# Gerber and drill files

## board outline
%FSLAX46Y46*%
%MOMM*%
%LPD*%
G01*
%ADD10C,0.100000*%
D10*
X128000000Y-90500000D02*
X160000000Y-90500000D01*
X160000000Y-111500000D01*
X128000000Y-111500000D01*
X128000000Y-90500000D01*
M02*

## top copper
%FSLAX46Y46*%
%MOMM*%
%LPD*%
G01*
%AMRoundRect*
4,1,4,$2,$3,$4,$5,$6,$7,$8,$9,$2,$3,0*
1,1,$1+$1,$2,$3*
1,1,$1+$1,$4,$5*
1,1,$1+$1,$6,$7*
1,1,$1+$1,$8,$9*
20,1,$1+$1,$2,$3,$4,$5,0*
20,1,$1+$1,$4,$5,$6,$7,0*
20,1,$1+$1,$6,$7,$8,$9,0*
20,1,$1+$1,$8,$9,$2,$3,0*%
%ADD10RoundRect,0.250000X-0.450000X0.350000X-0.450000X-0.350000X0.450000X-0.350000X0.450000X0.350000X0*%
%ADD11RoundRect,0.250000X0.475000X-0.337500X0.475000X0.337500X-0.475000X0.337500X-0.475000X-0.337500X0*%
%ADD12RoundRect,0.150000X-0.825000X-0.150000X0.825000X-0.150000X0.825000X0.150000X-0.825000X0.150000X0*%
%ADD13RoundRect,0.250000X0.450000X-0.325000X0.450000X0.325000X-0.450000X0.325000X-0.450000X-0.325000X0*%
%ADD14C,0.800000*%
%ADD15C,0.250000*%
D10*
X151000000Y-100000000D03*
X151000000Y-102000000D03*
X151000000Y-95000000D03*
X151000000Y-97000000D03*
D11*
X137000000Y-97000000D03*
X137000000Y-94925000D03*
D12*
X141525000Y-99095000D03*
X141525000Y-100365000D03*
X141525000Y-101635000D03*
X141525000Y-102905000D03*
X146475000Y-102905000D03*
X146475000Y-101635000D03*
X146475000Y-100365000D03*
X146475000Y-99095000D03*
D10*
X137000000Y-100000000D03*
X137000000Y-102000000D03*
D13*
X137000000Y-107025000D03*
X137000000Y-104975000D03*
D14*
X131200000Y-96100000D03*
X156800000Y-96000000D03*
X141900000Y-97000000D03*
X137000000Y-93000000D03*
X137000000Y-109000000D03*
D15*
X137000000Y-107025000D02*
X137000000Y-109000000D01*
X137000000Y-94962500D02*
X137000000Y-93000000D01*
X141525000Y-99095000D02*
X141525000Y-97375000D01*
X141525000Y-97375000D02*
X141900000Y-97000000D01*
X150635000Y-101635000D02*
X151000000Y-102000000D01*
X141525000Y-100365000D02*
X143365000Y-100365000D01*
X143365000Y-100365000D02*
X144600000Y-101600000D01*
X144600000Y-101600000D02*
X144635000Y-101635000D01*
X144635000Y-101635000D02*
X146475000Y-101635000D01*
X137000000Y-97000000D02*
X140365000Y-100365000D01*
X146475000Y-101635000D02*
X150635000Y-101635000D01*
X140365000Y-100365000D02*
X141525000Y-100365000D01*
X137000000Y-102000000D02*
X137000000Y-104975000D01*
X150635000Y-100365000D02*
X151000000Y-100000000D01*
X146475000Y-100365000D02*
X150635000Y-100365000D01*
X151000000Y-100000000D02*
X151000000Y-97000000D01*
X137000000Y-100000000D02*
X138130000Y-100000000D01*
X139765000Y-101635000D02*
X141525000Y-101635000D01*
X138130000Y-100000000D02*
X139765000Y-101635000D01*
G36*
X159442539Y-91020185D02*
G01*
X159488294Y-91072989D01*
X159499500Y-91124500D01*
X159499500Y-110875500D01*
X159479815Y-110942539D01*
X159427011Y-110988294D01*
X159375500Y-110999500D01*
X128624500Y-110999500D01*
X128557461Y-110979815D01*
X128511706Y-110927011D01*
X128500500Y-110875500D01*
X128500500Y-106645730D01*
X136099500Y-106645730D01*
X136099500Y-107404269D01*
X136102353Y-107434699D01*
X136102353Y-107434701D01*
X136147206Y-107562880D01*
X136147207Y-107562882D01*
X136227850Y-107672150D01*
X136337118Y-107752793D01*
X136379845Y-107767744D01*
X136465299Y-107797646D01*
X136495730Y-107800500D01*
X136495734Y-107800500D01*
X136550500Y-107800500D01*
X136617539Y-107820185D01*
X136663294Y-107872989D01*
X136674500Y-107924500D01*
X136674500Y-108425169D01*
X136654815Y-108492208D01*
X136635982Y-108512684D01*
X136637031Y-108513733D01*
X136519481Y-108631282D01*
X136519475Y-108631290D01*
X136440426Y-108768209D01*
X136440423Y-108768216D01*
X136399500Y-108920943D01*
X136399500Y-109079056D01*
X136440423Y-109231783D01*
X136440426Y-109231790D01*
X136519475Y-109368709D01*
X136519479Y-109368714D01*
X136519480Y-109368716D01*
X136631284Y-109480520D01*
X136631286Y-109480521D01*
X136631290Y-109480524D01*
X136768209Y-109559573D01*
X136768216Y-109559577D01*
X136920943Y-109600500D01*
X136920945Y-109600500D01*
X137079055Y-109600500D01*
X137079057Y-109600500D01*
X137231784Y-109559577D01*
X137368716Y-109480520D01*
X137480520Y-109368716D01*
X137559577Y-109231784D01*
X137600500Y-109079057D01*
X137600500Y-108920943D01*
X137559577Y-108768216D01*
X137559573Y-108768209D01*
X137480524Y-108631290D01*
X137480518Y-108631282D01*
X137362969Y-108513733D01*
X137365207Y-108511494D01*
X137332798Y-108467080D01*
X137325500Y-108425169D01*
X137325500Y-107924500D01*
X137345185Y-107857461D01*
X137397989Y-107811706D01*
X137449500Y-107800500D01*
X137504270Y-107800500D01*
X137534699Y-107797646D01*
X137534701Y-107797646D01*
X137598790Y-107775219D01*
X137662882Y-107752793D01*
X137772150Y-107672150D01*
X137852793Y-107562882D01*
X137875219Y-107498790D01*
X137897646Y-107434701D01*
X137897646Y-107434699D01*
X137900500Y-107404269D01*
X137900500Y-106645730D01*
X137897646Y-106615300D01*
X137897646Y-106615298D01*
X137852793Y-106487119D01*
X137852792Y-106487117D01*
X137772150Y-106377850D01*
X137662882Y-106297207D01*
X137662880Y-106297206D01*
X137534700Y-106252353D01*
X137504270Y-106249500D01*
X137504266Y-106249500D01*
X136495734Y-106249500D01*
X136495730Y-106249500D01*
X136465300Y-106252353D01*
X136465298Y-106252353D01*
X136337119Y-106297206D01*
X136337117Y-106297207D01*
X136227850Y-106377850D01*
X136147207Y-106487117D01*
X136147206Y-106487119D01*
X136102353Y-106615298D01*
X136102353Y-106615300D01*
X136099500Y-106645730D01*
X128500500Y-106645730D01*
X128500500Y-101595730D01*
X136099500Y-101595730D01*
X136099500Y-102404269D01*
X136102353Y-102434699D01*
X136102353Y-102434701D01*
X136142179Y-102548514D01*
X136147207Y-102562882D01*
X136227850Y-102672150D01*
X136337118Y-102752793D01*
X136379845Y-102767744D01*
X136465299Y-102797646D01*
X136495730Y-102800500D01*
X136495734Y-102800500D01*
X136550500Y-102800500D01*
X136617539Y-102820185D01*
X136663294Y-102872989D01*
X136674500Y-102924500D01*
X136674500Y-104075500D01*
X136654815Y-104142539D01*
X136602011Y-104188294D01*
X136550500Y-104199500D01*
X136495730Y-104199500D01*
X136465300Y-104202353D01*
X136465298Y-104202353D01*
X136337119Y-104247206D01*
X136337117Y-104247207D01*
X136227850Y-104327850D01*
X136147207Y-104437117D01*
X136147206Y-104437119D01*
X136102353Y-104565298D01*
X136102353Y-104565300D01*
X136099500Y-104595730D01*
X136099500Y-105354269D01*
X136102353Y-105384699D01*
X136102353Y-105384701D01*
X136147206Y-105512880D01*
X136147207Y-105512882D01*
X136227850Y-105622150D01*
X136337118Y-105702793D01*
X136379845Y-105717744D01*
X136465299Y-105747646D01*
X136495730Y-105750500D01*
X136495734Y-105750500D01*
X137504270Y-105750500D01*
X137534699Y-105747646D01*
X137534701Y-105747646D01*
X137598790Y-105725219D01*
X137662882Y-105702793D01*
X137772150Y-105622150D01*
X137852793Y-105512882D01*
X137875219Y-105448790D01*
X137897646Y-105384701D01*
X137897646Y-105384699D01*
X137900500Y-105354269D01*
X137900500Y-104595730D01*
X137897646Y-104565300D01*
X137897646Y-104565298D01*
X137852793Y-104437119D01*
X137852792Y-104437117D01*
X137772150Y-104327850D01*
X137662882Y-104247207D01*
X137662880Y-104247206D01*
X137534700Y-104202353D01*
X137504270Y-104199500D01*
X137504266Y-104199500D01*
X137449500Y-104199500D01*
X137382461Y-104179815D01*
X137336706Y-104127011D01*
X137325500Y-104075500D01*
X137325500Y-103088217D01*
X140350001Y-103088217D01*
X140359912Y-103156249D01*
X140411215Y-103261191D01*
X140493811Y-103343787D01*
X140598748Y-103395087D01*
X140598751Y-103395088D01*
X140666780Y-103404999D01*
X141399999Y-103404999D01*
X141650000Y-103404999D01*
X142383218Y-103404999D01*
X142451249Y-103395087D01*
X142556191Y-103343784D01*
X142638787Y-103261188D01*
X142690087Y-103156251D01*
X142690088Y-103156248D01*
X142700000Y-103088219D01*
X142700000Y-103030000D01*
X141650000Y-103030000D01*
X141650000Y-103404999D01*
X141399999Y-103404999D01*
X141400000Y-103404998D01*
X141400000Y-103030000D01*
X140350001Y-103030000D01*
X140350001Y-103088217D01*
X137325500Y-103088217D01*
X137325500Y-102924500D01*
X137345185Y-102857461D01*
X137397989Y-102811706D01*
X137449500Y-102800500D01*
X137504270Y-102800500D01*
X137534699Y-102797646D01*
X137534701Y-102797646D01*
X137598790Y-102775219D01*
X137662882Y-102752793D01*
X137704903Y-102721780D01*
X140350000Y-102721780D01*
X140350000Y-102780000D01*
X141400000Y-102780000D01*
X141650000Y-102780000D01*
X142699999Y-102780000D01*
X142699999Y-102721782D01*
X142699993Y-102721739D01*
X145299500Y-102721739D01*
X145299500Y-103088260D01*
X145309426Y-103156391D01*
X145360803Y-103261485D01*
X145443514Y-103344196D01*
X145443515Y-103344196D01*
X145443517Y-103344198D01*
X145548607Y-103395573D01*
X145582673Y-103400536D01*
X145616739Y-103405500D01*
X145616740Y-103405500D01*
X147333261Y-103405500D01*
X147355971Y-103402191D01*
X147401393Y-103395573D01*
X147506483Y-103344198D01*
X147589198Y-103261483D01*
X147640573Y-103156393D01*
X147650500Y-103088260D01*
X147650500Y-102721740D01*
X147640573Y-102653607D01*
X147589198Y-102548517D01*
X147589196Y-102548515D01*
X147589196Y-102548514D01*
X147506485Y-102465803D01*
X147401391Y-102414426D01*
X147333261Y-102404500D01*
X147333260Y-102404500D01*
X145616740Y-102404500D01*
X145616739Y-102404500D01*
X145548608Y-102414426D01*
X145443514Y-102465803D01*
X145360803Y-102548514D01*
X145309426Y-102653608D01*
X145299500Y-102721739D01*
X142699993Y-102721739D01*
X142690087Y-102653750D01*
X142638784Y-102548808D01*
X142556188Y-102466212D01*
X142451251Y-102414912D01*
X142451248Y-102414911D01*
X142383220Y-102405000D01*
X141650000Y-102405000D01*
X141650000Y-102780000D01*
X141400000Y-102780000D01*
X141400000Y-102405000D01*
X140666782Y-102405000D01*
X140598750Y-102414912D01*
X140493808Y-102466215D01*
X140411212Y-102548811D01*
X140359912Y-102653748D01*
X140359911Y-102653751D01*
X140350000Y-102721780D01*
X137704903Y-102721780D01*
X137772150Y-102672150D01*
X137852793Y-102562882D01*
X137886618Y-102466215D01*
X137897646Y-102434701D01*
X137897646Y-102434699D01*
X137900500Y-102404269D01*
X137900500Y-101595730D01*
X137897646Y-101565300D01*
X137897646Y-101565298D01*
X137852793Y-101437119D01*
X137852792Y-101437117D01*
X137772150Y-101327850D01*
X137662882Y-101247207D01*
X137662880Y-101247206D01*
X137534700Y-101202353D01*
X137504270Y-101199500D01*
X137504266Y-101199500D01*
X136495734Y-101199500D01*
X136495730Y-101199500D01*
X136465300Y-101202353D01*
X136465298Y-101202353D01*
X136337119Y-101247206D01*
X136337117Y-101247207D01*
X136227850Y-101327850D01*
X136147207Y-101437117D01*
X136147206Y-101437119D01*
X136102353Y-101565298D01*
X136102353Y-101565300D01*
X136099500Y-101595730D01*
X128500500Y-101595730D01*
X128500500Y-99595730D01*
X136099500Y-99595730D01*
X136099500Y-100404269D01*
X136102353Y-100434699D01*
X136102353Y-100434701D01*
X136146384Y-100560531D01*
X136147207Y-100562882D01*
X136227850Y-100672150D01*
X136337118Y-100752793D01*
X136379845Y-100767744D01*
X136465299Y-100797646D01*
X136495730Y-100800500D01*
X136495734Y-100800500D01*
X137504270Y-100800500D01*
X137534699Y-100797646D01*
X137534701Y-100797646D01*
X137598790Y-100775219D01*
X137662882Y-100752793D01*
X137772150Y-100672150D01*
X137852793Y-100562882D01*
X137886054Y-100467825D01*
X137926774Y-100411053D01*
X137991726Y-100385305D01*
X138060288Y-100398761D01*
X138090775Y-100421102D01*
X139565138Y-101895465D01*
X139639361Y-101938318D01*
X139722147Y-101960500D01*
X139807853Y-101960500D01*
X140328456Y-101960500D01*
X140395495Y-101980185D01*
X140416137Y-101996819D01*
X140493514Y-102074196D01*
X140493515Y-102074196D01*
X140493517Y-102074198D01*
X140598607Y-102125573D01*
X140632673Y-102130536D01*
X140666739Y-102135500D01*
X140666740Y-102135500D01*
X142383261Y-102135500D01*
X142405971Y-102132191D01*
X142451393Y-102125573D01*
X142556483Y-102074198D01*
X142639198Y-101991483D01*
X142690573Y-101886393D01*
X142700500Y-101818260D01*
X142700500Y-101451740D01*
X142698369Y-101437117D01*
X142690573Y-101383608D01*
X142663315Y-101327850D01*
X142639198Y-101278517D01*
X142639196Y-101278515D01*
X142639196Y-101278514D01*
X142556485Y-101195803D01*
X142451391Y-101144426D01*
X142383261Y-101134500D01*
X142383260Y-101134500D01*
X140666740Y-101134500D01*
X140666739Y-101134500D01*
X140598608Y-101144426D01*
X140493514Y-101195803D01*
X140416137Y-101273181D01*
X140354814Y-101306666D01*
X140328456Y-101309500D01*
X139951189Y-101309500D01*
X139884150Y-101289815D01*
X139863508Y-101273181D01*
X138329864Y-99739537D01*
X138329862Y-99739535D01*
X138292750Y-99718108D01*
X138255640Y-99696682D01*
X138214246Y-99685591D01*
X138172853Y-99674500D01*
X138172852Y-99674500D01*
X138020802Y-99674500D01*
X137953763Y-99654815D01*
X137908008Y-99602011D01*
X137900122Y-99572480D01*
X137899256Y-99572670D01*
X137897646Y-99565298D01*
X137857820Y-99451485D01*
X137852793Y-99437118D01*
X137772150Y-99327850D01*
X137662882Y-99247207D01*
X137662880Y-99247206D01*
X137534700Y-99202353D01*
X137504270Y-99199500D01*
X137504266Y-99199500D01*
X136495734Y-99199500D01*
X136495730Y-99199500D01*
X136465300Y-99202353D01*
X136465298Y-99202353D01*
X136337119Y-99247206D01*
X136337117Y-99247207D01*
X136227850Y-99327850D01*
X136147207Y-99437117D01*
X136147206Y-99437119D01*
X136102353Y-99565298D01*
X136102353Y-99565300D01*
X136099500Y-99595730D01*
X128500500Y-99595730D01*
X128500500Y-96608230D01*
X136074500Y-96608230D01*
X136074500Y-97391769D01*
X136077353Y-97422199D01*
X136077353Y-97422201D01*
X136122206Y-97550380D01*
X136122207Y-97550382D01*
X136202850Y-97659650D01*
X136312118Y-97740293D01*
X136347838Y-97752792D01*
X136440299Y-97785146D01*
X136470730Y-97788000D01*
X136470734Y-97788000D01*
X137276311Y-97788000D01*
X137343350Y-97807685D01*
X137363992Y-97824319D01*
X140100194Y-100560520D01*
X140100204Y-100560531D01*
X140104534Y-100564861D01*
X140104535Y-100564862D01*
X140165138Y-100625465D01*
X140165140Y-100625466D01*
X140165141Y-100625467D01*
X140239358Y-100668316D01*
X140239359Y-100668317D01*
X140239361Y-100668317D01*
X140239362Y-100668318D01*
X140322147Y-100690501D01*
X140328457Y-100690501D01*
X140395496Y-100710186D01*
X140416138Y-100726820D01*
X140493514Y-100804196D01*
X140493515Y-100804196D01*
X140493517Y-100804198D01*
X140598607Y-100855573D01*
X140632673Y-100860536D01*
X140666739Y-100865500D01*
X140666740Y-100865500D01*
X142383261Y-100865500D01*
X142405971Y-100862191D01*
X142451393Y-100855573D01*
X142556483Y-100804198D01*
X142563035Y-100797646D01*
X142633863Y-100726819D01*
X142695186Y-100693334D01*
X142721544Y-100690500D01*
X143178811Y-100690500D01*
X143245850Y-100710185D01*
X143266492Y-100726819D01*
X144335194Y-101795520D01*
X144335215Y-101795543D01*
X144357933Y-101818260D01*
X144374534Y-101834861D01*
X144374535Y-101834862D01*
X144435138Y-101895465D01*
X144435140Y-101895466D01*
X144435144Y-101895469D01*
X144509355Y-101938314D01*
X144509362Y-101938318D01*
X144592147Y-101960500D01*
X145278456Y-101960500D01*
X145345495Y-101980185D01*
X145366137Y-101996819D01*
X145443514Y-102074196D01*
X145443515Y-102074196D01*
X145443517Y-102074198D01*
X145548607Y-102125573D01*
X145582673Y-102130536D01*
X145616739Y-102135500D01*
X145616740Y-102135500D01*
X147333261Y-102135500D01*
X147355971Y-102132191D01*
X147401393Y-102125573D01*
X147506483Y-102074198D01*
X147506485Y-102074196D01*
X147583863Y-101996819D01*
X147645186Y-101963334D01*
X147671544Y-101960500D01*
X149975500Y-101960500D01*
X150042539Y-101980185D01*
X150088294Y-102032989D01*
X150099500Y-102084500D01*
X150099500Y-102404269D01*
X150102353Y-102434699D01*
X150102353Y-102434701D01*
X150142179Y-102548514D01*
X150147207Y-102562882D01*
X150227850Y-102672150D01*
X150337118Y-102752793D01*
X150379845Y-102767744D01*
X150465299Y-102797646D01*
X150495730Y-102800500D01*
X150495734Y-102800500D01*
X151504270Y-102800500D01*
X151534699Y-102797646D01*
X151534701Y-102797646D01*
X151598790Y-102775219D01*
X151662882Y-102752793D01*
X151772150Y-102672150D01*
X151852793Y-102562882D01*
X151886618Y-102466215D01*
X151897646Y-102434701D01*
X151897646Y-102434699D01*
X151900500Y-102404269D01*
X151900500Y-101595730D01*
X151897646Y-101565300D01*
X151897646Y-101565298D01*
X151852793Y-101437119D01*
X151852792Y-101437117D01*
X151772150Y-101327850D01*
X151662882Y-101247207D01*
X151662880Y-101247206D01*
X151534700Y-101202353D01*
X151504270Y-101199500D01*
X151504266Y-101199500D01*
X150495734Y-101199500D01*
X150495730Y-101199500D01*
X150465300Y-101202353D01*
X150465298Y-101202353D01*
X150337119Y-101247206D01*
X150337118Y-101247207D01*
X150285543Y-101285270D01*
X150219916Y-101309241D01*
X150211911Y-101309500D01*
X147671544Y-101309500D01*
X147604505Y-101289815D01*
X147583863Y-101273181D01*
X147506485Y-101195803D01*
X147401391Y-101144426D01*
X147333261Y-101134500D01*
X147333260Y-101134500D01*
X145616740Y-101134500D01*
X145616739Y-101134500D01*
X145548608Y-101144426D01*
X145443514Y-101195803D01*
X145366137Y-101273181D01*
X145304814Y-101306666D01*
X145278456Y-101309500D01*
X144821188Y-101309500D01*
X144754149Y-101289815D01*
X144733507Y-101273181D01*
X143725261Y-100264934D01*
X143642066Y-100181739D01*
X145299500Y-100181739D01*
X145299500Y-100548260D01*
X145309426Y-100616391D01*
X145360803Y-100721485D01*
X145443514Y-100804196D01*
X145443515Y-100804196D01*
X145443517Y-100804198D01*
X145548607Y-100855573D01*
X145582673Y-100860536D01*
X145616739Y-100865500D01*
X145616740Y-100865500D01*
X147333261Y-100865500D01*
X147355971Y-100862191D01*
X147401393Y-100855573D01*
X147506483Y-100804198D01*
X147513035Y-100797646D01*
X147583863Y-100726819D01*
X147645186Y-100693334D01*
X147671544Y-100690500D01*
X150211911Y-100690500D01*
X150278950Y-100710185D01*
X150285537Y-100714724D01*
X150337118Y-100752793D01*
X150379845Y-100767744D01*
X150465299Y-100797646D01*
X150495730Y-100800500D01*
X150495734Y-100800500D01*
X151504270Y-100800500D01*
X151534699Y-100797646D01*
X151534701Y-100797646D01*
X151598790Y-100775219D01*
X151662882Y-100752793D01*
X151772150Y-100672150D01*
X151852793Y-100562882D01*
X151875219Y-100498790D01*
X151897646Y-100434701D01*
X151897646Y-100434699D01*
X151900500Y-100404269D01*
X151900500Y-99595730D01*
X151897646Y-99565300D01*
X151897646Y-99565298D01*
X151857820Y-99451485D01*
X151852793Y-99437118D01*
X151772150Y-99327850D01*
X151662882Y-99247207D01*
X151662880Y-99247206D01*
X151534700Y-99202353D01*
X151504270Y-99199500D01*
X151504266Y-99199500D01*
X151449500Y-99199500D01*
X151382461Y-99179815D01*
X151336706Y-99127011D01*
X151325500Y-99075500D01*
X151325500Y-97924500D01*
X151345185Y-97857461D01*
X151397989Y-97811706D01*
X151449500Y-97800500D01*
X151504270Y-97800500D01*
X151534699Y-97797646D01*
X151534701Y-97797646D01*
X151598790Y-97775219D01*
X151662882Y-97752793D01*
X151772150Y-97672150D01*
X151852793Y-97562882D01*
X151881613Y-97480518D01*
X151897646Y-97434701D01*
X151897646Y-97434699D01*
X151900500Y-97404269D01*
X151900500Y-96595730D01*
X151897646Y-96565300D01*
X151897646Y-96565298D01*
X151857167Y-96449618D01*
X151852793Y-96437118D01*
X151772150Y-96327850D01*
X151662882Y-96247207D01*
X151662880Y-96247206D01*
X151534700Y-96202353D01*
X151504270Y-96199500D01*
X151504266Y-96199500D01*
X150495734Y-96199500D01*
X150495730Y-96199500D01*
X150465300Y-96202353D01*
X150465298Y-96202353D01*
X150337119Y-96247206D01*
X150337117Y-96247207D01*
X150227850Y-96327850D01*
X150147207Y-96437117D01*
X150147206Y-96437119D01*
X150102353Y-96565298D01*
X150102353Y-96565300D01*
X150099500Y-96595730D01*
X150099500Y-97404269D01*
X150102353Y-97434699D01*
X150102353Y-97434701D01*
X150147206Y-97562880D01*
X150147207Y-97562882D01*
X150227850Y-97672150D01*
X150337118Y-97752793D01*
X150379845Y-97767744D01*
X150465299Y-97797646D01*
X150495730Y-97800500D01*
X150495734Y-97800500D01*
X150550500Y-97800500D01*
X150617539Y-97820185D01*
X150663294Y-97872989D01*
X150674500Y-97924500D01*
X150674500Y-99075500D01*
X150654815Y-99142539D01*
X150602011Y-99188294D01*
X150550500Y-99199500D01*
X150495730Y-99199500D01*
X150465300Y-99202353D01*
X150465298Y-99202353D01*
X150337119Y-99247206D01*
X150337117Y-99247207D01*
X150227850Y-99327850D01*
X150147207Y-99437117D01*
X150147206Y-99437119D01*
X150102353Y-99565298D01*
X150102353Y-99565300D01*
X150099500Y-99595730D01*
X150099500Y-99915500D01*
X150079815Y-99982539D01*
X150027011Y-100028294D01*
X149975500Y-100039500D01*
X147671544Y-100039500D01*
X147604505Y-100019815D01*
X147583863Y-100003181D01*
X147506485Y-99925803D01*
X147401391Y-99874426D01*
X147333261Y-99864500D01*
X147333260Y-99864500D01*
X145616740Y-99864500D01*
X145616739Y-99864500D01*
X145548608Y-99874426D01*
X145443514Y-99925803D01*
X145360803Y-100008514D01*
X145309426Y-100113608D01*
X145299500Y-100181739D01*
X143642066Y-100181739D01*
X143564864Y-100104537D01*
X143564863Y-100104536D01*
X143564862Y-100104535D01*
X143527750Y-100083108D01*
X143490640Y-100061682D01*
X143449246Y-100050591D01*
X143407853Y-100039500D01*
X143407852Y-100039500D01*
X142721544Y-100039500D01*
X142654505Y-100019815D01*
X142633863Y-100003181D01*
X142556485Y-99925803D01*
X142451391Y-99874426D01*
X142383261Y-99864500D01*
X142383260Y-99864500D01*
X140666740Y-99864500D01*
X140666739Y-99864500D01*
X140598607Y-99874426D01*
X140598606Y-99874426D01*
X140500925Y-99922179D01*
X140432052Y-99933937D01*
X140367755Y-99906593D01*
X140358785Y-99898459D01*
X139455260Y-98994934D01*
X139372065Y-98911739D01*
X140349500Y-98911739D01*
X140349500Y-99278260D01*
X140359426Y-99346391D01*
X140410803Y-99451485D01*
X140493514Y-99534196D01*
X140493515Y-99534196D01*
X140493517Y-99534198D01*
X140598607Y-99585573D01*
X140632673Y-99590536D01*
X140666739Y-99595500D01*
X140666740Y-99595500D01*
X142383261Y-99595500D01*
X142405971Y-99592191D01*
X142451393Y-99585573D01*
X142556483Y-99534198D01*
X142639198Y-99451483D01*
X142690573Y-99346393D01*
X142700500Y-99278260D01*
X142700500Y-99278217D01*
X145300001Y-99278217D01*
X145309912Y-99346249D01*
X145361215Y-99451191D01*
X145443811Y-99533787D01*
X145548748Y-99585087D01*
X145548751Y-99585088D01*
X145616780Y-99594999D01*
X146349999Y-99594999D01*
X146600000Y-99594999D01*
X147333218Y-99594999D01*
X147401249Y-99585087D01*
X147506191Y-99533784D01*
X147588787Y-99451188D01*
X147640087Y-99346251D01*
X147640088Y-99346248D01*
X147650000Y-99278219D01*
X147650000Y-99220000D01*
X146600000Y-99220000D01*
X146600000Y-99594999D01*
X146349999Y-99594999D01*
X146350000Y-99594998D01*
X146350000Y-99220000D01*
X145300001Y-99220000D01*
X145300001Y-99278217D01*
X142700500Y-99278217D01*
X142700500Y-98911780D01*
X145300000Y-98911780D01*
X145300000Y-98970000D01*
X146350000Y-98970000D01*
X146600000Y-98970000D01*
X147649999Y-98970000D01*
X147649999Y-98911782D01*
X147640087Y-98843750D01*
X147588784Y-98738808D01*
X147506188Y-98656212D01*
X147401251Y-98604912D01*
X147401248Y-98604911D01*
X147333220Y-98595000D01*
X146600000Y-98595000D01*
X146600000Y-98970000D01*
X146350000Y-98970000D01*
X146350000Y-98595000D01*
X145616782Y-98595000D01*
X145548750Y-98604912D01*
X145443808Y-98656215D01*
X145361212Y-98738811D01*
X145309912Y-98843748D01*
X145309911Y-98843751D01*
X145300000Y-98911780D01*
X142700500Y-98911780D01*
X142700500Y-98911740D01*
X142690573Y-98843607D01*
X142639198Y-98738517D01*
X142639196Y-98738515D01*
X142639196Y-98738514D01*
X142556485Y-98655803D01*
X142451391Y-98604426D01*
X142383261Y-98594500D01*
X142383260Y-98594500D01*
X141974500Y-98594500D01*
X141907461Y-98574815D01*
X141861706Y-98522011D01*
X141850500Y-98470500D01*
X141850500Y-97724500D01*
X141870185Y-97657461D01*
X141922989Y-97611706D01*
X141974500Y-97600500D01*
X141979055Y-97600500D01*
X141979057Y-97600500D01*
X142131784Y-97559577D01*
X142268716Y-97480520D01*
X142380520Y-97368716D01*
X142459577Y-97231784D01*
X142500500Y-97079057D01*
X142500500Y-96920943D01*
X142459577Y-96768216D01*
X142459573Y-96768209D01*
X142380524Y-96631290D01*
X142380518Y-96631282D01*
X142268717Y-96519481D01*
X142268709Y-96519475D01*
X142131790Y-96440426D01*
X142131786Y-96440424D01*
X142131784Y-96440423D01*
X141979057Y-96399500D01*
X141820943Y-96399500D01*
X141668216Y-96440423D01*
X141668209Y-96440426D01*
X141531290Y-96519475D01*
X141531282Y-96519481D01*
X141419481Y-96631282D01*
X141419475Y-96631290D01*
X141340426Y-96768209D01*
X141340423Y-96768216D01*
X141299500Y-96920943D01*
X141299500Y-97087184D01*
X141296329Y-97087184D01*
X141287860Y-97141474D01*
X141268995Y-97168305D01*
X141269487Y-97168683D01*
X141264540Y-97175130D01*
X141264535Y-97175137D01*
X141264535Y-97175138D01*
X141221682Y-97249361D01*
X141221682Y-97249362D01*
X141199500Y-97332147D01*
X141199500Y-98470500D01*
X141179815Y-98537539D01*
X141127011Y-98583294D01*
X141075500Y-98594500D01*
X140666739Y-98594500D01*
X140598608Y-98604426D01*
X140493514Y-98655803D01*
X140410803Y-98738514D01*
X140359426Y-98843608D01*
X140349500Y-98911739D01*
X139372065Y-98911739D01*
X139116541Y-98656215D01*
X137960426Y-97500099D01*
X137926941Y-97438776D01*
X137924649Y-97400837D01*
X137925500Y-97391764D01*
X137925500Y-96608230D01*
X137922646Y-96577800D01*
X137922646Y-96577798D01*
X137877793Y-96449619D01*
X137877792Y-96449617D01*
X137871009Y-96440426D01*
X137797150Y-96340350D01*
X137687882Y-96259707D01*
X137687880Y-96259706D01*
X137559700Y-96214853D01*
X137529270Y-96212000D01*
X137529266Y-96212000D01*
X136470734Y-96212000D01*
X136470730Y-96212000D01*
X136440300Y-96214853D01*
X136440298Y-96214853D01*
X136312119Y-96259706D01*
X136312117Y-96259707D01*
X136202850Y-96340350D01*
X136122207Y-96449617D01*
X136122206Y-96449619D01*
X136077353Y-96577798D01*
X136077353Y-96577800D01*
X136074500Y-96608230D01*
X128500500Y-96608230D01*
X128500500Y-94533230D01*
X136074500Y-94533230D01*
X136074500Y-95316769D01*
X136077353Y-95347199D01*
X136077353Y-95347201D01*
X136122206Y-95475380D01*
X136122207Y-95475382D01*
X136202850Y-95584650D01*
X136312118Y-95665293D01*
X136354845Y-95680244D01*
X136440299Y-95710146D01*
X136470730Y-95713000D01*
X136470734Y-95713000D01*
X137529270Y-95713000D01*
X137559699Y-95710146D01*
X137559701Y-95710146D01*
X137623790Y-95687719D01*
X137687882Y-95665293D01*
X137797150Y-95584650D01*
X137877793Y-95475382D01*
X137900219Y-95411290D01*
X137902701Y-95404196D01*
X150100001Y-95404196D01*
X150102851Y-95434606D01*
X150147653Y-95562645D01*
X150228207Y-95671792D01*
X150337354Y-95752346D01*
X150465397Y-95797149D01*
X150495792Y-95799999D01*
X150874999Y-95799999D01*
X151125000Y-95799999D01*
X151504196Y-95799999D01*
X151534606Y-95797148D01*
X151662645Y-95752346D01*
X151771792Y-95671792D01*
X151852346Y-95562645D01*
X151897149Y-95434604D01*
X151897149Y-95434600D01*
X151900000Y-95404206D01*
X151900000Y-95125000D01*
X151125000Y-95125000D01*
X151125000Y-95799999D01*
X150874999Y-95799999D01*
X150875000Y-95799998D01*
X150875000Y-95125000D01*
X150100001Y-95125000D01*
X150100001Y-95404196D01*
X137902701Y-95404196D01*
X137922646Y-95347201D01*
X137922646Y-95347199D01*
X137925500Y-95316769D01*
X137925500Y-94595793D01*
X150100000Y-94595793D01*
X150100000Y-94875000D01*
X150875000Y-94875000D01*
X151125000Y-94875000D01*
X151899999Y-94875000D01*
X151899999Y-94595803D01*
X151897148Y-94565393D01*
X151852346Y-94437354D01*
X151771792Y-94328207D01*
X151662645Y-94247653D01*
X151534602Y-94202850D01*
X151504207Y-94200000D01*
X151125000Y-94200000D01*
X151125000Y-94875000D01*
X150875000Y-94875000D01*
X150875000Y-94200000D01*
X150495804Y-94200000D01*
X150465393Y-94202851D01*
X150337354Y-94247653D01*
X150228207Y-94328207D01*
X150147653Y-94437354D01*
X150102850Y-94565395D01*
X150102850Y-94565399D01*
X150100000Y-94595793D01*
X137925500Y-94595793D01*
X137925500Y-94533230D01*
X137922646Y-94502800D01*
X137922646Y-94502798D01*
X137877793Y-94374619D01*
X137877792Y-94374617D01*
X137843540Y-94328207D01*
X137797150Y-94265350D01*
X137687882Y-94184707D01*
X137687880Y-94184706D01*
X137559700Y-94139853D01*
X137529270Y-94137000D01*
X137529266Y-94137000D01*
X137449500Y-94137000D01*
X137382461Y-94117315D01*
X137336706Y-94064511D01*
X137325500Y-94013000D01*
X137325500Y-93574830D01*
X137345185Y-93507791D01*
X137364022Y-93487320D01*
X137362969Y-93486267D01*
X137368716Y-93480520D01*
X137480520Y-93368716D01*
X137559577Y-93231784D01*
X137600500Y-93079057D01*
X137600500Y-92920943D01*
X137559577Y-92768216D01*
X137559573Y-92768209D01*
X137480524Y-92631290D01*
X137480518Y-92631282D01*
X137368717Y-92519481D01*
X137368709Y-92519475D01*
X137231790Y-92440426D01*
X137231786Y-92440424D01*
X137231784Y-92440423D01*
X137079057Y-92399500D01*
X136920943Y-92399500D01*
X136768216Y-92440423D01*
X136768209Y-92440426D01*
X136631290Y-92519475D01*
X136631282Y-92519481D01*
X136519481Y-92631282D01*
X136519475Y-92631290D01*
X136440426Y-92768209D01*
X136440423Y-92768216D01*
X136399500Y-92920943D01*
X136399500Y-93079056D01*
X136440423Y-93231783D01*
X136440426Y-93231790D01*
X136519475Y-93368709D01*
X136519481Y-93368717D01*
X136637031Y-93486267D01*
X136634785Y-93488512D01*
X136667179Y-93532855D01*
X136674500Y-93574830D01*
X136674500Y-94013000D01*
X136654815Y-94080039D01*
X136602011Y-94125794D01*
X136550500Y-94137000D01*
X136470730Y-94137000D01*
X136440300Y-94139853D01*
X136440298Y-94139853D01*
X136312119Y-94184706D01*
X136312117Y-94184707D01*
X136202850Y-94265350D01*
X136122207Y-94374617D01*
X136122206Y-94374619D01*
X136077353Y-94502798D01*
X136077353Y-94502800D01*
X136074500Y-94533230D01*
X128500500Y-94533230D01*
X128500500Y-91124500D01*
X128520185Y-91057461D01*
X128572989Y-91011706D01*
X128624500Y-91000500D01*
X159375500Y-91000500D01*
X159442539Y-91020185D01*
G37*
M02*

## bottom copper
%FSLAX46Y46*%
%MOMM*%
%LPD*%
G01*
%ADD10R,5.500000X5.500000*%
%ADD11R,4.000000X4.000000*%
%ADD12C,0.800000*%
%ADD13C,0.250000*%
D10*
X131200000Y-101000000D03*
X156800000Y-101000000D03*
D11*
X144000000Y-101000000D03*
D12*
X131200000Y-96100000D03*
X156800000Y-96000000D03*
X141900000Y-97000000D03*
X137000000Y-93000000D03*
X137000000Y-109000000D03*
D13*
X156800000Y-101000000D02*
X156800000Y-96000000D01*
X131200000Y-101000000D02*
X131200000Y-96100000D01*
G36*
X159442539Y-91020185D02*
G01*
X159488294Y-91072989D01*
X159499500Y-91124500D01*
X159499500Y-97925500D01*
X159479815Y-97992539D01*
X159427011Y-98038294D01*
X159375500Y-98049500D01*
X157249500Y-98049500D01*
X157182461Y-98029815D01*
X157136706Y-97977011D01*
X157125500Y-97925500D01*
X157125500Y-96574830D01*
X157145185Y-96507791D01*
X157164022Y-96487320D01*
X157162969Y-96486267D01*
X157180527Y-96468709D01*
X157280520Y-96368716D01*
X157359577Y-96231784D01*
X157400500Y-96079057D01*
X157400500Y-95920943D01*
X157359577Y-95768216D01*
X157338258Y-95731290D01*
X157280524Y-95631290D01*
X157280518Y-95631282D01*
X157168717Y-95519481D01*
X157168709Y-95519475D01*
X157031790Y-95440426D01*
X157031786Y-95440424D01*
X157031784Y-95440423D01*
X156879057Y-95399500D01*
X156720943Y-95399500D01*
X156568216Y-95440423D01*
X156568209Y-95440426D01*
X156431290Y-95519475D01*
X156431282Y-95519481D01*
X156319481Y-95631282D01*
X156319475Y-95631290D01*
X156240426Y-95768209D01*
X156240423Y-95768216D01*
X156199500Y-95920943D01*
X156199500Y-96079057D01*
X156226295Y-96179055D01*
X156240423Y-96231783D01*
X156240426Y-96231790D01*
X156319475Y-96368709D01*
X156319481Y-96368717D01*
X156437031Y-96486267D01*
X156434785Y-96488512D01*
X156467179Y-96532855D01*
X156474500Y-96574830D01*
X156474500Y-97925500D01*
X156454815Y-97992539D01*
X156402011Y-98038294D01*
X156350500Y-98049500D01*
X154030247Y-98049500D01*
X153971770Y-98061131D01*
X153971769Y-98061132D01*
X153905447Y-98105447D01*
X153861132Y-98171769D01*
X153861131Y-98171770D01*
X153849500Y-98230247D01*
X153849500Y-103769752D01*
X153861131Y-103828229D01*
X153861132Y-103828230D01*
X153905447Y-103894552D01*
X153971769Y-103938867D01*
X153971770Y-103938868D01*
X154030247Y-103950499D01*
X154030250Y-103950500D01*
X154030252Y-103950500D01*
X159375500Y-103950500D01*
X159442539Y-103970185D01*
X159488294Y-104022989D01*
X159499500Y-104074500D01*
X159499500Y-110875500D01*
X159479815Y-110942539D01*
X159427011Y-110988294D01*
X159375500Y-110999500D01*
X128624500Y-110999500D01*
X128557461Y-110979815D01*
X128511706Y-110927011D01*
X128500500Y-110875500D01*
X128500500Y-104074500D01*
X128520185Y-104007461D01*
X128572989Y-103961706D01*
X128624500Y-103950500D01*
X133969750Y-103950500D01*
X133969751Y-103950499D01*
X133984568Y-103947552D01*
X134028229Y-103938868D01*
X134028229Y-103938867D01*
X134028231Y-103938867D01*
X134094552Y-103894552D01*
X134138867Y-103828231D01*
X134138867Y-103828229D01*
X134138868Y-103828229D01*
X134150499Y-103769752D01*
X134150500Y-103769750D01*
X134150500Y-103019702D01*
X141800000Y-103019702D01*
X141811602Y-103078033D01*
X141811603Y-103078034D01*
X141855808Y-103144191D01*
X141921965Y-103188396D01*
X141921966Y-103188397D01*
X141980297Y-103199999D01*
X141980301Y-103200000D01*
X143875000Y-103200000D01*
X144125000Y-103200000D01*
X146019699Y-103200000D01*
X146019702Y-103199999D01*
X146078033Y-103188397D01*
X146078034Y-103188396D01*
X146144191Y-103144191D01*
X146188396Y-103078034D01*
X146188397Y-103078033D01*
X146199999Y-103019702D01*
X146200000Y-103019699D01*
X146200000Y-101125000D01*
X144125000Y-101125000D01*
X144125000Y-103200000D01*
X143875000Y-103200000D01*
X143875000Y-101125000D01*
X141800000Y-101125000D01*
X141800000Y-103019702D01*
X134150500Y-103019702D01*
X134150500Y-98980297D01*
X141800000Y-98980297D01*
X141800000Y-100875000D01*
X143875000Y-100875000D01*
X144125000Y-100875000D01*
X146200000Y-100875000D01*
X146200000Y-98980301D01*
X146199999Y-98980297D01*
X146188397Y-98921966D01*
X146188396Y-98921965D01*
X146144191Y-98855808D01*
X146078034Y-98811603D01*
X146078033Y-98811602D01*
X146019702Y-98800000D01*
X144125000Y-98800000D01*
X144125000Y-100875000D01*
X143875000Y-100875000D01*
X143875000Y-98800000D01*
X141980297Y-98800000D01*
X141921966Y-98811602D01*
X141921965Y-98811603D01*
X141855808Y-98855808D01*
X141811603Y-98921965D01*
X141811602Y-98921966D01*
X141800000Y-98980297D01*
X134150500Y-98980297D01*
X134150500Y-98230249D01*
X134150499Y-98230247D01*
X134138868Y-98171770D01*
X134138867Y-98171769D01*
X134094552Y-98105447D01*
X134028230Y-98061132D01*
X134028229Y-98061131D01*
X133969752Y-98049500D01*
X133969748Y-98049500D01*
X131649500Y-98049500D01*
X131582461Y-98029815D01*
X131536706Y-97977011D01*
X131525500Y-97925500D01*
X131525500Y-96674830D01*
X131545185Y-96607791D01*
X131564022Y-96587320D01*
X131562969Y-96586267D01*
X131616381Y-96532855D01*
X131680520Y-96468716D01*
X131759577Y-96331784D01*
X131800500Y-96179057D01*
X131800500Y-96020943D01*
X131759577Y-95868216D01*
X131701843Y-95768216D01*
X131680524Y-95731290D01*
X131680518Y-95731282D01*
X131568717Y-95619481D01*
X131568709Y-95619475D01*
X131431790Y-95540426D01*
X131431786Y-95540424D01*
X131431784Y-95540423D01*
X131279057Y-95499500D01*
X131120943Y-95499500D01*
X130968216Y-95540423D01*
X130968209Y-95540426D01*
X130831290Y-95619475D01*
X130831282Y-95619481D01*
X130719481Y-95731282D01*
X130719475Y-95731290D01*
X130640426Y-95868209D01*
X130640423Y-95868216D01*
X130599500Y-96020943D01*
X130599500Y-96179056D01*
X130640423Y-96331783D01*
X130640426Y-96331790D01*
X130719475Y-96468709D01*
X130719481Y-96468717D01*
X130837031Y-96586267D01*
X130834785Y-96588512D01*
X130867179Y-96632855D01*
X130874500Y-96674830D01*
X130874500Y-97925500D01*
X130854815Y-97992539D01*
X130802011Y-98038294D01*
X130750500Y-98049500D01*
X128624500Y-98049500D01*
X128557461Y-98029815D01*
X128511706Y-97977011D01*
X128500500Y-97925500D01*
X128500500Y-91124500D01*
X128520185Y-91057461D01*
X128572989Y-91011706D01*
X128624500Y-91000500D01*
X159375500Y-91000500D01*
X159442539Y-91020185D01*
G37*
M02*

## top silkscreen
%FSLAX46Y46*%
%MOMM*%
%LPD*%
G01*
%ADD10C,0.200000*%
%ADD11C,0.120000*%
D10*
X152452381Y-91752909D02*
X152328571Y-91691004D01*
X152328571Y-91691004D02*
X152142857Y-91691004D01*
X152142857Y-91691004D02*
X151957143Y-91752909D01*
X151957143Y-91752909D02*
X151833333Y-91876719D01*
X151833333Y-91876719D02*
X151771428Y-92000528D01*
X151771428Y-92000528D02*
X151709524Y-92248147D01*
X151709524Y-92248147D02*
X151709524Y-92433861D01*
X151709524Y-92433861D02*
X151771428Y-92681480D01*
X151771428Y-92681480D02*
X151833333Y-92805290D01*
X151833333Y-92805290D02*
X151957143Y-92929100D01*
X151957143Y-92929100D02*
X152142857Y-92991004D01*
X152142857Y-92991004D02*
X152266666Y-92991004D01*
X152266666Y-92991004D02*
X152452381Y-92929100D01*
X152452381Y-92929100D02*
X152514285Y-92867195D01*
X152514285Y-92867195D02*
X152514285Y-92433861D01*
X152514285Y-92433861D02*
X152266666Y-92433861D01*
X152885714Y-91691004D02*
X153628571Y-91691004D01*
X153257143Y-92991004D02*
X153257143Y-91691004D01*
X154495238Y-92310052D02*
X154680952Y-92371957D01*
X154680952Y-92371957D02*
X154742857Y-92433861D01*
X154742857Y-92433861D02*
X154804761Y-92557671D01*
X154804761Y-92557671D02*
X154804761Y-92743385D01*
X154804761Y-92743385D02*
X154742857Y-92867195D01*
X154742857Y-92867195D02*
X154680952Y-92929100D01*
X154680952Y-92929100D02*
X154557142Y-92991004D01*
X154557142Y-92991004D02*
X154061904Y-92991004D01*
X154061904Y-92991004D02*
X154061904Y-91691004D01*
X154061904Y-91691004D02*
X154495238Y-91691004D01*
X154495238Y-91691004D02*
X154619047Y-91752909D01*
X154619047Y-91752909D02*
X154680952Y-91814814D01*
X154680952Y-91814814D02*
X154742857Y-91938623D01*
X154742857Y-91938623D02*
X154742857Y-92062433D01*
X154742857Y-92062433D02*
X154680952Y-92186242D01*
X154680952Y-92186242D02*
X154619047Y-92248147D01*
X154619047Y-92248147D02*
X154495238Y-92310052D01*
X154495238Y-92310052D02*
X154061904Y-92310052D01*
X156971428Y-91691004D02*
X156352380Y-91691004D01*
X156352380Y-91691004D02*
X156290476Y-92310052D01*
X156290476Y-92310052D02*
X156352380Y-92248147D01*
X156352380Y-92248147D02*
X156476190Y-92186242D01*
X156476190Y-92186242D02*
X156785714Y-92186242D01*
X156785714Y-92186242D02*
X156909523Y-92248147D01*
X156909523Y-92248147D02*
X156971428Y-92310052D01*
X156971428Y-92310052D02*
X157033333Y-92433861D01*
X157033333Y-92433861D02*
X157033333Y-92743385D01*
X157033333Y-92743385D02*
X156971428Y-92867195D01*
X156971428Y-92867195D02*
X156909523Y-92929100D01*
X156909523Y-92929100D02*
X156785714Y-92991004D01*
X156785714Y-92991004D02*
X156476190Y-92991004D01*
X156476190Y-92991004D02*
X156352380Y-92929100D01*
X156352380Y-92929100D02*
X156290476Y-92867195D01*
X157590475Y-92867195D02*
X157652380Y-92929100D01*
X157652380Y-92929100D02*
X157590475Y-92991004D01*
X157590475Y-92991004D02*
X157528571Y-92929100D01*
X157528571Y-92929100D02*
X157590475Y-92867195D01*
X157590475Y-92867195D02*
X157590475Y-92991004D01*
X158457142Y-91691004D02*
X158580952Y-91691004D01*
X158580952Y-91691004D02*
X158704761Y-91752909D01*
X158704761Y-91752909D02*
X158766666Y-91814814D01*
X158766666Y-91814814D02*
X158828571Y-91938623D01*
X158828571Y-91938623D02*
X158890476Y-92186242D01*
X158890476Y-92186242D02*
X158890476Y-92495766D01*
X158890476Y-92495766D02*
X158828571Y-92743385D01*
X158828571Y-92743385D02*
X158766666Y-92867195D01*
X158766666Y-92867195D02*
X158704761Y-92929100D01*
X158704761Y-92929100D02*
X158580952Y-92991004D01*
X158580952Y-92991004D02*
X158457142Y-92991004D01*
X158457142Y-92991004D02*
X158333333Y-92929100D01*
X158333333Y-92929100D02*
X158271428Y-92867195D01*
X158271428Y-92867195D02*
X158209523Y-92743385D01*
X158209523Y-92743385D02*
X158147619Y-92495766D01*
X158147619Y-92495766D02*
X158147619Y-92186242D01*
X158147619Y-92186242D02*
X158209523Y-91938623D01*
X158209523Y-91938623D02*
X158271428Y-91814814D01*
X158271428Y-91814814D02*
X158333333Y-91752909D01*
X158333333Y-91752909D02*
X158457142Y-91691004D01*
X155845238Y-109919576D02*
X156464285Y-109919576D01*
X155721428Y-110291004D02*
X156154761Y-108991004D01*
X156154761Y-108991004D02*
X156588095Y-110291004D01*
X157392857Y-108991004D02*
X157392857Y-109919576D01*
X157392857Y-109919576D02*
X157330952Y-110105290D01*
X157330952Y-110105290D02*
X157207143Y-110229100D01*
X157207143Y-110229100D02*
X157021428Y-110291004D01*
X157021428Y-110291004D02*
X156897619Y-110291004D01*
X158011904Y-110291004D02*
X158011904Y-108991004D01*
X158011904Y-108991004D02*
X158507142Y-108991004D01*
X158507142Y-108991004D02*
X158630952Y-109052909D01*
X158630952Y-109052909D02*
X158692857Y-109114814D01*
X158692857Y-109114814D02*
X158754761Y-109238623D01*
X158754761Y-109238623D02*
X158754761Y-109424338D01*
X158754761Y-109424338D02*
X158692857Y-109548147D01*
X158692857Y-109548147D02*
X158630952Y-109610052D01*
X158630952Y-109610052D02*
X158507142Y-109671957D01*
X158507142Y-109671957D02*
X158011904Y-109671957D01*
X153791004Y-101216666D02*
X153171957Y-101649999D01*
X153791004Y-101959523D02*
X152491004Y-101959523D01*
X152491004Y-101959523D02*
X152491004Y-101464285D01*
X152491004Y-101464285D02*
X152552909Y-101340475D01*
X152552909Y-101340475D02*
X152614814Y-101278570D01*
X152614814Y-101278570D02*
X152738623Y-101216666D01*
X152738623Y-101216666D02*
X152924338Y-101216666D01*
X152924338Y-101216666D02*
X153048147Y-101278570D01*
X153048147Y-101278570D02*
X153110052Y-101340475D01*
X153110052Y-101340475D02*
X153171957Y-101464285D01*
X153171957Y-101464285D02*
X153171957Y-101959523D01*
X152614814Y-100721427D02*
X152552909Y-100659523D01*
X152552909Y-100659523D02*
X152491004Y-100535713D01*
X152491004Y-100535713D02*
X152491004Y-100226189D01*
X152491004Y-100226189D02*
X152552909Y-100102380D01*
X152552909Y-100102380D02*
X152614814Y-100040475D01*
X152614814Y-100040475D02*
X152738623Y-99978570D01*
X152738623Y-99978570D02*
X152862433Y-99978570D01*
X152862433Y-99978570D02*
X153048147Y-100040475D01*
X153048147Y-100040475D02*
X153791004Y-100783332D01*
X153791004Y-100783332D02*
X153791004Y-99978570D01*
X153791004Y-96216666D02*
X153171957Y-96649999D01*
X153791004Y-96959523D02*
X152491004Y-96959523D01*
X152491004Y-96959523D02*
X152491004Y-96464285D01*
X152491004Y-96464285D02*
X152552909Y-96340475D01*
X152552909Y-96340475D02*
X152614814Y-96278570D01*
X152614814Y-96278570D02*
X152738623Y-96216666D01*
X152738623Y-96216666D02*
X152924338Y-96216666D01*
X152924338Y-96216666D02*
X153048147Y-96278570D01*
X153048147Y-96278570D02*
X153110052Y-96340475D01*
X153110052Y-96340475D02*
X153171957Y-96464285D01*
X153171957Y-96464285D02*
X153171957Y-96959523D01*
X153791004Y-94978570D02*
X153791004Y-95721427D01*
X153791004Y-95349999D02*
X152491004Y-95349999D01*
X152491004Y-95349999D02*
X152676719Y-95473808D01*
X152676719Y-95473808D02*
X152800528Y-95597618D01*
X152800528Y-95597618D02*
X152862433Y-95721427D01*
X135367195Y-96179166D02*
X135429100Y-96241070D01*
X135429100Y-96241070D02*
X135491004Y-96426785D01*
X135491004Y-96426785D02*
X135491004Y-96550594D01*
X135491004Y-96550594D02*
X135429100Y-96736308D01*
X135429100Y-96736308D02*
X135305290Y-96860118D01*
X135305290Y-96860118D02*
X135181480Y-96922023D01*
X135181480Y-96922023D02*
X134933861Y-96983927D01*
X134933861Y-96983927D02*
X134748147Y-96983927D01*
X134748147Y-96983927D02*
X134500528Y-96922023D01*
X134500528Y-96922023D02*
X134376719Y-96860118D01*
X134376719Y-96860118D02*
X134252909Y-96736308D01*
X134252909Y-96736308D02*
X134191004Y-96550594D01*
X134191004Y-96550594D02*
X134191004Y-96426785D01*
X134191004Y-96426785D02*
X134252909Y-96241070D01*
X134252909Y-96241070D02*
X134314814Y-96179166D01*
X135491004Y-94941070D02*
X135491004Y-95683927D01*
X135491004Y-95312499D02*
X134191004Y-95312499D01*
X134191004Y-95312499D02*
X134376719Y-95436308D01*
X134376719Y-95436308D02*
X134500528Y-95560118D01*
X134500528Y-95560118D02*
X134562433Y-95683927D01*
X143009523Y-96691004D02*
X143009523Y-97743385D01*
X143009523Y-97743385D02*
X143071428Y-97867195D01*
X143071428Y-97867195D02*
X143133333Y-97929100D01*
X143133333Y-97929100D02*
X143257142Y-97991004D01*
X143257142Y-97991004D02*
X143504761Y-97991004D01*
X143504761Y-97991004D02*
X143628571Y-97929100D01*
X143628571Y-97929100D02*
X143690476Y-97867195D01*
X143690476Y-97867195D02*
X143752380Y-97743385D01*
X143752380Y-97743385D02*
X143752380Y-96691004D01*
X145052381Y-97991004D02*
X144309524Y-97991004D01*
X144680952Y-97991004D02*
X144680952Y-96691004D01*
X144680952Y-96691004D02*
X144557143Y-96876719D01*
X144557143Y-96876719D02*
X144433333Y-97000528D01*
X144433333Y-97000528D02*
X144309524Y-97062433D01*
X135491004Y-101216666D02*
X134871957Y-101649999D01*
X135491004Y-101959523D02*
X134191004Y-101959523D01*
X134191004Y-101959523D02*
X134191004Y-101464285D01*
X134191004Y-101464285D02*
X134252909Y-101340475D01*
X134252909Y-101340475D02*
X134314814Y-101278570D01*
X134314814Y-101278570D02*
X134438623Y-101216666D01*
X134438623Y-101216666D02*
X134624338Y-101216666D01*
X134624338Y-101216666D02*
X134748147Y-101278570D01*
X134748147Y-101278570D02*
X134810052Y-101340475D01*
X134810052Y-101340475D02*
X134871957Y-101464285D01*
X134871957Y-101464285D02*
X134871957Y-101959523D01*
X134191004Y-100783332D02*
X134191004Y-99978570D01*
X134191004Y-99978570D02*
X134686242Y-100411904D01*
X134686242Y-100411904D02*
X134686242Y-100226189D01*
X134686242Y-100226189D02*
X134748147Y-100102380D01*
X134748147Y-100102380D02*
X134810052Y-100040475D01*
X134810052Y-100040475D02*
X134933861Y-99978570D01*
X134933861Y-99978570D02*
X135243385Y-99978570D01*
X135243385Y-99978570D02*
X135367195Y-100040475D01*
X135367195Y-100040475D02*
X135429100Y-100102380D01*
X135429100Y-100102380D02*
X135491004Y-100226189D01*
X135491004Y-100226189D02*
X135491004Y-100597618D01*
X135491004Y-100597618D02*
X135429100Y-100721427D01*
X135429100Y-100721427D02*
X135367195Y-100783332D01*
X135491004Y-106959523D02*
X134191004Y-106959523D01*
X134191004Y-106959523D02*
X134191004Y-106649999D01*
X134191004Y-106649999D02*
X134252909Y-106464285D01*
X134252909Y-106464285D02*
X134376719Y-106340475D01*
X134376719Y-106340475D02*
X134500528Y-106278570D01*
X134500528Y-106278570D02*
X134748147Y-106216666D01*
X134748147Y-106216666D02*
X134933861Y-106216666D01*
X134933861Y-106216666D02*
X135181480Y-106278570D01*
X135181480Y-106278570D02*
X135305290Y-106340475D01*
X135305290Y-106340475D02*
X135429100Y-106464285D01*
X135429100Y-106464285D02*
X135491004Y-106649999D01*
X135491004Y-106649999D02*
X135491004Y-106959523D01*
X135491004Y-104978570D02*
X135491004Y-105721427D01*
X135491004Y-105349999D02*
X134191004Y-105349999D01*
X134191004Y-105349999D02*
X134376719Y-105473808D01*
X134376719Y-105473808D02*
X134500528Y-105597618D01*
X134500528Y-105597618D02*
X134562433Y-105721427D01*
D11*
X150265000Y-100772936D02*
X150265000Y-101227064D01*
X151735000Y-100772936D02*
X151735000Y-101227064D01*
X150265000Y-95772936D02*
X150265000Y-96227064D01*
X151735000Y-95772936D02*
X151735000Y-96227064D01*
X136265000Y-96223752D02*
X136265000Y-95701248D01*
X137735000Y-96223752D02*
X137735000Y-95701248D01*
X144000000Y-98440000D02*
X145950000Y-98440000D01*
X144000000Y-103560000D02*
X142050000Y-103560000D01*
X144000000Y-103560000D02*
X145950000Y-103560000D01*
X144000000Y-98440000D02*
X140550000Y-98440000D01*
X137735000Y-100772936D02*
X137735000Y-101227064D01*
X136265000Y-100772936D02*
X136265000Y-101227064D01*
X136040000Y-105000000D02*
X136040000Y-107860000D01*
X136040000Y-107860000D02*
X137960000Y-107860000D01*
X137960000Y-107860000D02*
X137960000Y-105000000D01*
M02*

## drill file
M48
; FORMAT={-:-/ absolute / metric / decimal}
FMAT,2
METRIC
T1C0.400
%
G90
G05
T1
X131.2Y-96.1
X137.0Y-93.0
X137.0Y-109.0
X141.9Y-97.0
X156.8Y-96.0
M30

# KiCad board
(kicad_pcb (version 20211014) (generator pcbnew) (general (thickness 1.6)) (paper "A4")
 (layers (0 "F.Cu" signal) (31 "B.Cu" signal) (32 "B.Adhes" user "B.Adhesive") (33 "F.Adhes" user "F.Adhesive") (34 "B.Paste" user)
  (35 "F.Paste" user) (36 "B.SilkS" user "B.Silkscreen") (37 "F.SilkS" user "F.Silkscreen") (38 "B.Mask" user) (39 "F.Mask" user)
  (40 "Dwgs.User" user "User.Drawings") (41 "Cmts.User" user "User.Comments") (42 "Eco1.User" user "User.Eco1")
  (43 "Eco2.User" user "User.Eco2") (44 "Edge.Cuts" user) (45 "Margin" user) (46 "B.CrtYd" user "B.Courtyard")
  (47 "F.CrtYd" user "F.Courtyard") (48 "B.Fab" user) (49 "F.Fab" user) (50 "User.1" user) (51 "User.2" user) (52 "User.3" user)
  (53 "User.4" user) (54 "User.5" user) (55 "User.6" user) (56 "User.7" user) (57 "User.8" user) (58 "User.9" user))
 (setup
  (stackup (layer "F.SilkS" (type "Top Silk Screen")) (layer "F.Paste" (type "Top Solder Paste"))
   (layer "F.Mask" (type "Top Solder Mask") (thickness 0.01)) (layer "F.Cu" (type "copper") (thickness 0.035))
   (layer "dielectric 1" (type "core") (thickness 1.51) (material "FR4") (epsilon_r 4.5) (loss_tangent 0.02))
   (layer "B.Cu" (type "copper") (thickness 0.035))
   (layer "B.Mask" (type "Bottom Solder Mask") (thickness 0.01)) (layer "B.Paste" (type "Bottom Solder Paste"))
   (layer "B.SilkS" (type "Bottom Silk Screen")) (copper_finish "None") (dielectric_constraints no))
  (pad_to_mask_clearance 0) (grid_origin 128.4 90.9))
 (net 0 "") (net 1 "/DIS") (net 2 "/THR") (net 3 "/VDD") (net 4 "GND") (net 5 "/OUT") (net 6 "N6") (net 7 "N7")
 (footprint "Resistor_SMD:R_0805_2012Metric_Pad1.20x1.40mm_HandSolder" (layer "F.Cu") (at 151 101 -90)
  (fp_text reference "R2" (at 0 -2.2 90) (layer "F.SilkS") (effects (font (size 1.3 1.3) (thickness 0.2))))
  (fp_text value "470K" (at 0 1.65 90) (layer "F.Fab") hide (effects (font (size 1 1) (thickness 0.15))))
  (fp_line (start -0.227064 0.735) (end 0.227064 0.735) (layer "F.SilkS") (width 0.12))
  (fp_line (start -0.227064 -0.735) (end 0.227064 -0.735) (layer "F.SilkS") (width 0.12))
  (pad "1" smd roundrect (at -1 0 270) (size 1.2 1.4) (layers "F.Cu" "F.Paste" "F.Mask") (roundrect_rratio 0.208333) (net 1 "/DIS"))
  (pad "2" smd roundrect (at 1 0 270) (size 1.2 1.4) (layers "F.Cu" "F.Paste" "F.Mask") (roundrect_rratio 0.208333) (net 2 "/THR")))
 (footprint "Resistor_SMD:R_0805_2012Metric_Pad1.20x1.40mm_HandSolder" (layer "F.Cu") (at 151 96 -90)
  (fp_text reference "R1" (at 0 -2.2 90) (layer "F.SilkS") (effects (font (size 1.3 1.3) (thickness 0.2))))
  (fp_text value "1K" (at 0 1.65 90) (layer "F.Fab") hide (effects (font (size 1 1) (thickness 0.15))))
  (fp_line (start -0.227064 0.735) (end 0.227064 0.735) (layer "F.SilkS") (width 0.12))
  (fp_line (start -0.227064 -0.735) (end 0.227064 -0.735) (layer "F.SilkS") (width 0.12))
  (pad "1" smd roundrect (at -1 0 270) (size 1.2 1.4) (layers "F.Cu" "F.Paste" "F.Mask") (roundrect_rratio 0.208333) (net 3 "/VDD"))
  (pad "2" smd roundrect (at 1 0 270) (size 1.2 1.4) (layers "F.Cu" "F.Paste" "F.Mask") (roundrect_rratio 0.208333) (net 1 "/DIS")))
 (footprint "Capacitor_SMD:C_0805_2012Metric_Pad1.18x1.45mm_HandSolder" (layer "F.Cu") (at 137 95.9625 90)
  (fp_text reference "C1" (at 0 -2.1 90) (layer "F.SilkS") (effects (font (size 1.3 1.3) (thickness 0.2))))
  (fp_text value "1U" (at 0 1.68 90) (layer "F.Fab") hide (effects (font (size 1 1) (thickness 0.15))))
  (fp_line (start -0.261252 -0.735) (end 0.261252 -0.735) (layer "F.SilkS") (width 0.12))
  (fp_line (start -0.261252 0.735) (end 0.261252 0.735) (layer "F.SilkS") (width 0.12))
  (pad "1" smd roundrect (at -1.0375 0 90) (size 1.175 1.45) (layers "F.Cu" "F.Paste" "F.Mask") (roundrect_rratio 0.212766) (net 2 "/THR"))
  (pad "2" smd roundrect (at 1.0375 0 90) (size 1.175 1.45) (layers "F.Cu" "F.Paste" "F.Mask") (roundrect_rratio 0.212766) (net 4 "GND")))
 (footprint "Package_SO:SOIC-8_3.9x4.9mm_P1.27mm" (layer "F.Cu") (at 144 101)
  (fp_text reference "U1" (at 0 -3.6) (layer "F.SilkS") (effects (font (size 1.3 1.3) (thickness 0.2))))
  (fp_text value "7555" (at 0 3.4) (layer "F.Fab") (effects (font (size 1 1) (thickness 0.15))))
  (fp_line (start 0 -2.56) (end 1.95 -2.56) (layer "F.SilkS") (width 0.12))
  (fp_line (start 0 2.56) (end -1.95 2.56) (layer "F.SilkS") (width 0.12))
  (fp_line (start 0 2.56) (end 1.95 2.56) (layer "F.SilkS") (width 0.12))
  (fp_line (start 0 -2.56) (end -3.45 -2.56) (layer "F.SilkS") (width 0.12))
  (pad "1" smd roundrect (at -2.475 -1.905) (size 1.95 0.6) (layers "F.Cu" "F.Paste" "F.Mask") (roundrect_rratio 0.25) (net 4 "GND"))
  (pad "2" smd roundrect (at -2.475 -0.635) (size 1.95 0.6) (layers "F.Cu" "F.Paste" "F.Mask") (roundrect_rratio 0.25) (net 2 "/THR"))
  (pad "3" smd roundrect (at -2.475 0.635) (size 1.95 0.6) (layers "F.Cu" "F.Paste" "F.Mask") (roundrect_rratio 0.25) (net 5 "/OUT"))
  (pad "4" smd roundrect (at -2.475 1.905) (size 1.95 0.6) (layers "F.Cu" "F.Paste" "F.Mask") (roundrect_rratio 0.25) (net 3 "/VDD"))
  (pad "5" smd roundrect (at 2.475 1.905) (size 1.95 0.6) (layers "F.Cu" "F.Paste" "F.Mask") (roundrect_rratio 0.25) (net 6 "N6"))
  (pad "6" smd roundrect (at 2.475 0.635) (size 1.95 0.6) (layers "F.Cu" "F.Paste" "F.Mask") (roundrect_rratio 0.25) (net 2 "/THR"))
  (pad "7" smd roundrect (at 2.475 -0.635) (size 1.95 0.6) (layers "F.Cu" "F.Paste" "F.Mask") (roundrect_rratio 0.25) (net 1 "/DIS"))
  (pad "8" smd roundrect (at 2.475 -1.905) (size 1.95 0.6) (layers "F.Cu" "F.Paste" "F.Mask") (roundrect_rratio 0.25) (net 3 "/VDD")))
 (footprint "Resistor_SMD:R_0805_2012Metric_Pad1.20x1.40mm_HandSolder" (layer "F.Cu") (at 137 101 -90)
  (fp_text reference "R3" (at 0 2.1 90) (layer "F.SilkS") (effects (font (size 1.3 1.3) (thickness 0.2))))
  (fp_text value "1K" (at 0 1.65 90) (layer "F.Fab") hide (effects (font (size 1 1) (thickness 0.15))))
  (fp_line (start -0.227064 -0.735) (end 0.227064 -0.735) (layer "F.SilkS") (width 0.12))
  (fp_line (start -0.227064 0.735) (end 0.227064 0.735) (layer "F.SilkS") (width 0.12))
  (pad "1" smd roundrect (at -1 0 270) (size 1.2 1.4) (layers "F.Cu" "F.Paste" "F.Mask") (roundrect_rratio 0.208333) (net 5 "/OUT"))
  (pad "2" smd roundrect (at 1 0 270) (size 1.2 1.4) (layers "F.Cu" "F.Paste" "F.Mask") (roundrect_rratio 0.208333) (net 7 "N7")))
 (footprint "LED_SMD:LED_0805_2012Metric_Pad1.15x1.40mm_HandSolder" (layer "F.Cu") (at 137 106 90)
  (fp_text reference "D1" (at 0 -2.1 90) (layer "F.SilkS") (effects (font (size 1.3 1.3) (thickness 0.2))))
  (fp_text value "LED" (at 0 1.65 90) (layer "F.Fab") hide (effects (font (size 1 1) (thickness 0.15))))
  (fp_line (start 1 -0.96) (end -1.86 -0.96) (layer "F.SilkS") (width 0.12))
  (fp_line (start -1.86 -0.96) (end -1.86 0.96) (layer "F.SilkS") (width 0.12))
  (fp_line (start -1.86 0.96) (end 1 0.96) (layer "F.SilkS") (width 0.12))
  (pad "1" smd roundrect (at -1.025 0 90) (size 1.15 1.4) (layers "F.Cu" "F.Paste" "F.Mask") (roundrect_rratio 0.217391) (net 4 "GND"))
  (pad "2" smd roundrect (at 1.025 0 90) (size 1.15 1.4) (layers "F.Cu" "F.Paste" "F.Mask") (roundrect_rratio 0.217391) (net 7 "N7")))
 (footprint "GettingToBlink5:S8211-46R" (layer "B.Cu") (at 144 101 180)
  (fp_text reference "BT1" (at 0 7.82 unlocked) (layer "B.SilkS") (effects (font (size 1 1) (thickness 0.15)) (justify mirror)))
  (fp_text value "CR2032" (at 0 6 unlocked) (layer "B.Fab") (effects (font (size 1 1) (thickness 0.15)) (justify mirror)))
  (pad "1" smd rect (at 12.8 0 180) (size 5.5 5.5) (layers "B.Cu" "B.Paste" "B.Mask") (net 3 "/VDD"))
  (pad "1" smd rect (at -12.8 0 180) (size 5.5 5.5) (layers "B.Cu" "B.Paste" "B.Mask") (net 3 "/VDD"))
  (pad "2" smd rect (at 0 0 180) (size 4 4) (layers "B.Cu" "B.Paste" "B.Mask") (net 4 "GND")))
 (gr_rect (start 160 111.5) (end 128 90.5) (layer "Edge.Cuts") (width 0.1) (fill none))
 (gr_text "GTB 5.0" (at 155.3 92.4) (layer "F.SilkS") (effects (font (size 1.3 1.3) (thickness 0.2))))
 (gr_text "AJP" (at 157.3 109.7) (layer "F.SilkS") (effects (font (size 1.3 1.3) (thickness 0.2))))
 (via (at 131.2 96.1) (size 0.8) (drill 0.4) (layers "F.Cu" "B.Cu") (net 3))
 (via (at 156.8 96) (size 0.8) (drill 0.4) (layers "F.Cu" "B.Cu") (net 3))
 (segment (start 156.8 101) (end 156.8 96) (width 0.25) (layer "B.Cu") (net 3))
 (segment (start 131.2 101) (end 131.2 96.1) (width 0.25) (layer "B.Cu") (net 3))
 (segment (start 137 107.025) (end 137 109) (width 0.25) (layer "F.Cu") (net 4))
 (segment (start 137 94.9625) (end 137 93) (width 0.25) (layer "F.Cu") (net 4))
 (segment (start 141.525 99.095) (end 141.525 97.375) (width 0.25) (layer "F.Cu") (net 4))
 (segment (start 141.525 97.375) (end 141.9 97) (width 0.25) (layer "F.Cu") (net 4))
 (via (at 141.9 97) (size 0.8) (drill 0.4) (layers "F.Cu" "B.Cu") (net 4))
 (via (at 137 93) (size 0.8) (drill 0.4) (layers "F.Cu" "B.Cu") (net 4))
 (via (at 137 109) (size 0.8) (drill 0.4) (layers "F.Cu" "B.Cu") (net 4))
 (segment (start 150.635 101.635) (end 151 102) (width 0.25) (layer "F.Cu") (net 2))
 (segment (start 141.525 100.365) (end 143.365 100.365) (width 0.25) (layer "F.Cu") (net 2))
 (segment (start 143.365 100.365) (end 144.6 101.6) (width 0.25) (layer "F.Cu") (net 2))
 (segment (start 144.6 101.6) (end 144.635 101.635) (width 0.25) (layer "F.Cu") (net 2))
 (segment (start 144.635 101.635) (end 146.475 101.635) (width 0.25) (layer "F.Cu") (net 2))
 (segment (start 137 97) (end 140.365 100.365) (width 0.25) (layer "F.Cu") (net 2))
 (segment (start 146.475 101.635) (end 150.635 101.635) (width 0.25) (layer "F.Cu") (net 2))
 (segment (start 140.365 100.365) (end 141.525 100.365) (width 0.25) (layer "F.Cu") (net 2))
 (segment (start 137 102) (end 137 104.975) (width 0.25) (layer "F.Cu") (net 7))
 (segment (start 150.635 100.365) (end 151 100) (width 0.25) (layer "F.Cu") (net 1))
 (segment (start 146.475 100.365) (end 150.635 100.365) (width 0.25) (layer "F.Cu") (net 1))
 (segment (start 151 100) (end 151 97) (width 0.25) (layer "F.Cu") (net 1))
 (segment (start 137 100) (end 138.13 100) (width 0.25) (layer "F.Cu") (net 5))
 (segment (start 139.765 101.635) (end 141.525 101.635) (width 0.25) (layer "F.Cu") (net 5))
 (segment (start 138.13 100) (end 139.765 101.635) (width 0.25) (layer "F.Cu") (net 5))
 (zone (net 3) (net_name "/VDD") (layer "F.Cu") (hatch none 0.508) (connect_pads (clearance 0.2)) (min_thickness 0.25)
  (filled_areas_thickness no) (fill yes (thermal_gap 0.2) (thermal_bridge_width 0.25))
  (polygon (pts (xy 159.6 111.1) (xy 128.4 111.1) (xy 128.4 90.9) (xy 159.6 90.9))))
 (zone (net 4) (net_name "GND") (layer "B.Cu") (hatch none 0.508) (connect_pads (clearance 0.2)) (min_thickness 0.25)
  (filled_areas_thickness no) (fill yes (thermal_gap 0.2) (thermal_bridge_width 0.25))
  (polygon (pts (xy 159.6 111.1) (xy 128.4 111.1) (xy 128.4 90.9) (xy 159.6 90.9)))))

